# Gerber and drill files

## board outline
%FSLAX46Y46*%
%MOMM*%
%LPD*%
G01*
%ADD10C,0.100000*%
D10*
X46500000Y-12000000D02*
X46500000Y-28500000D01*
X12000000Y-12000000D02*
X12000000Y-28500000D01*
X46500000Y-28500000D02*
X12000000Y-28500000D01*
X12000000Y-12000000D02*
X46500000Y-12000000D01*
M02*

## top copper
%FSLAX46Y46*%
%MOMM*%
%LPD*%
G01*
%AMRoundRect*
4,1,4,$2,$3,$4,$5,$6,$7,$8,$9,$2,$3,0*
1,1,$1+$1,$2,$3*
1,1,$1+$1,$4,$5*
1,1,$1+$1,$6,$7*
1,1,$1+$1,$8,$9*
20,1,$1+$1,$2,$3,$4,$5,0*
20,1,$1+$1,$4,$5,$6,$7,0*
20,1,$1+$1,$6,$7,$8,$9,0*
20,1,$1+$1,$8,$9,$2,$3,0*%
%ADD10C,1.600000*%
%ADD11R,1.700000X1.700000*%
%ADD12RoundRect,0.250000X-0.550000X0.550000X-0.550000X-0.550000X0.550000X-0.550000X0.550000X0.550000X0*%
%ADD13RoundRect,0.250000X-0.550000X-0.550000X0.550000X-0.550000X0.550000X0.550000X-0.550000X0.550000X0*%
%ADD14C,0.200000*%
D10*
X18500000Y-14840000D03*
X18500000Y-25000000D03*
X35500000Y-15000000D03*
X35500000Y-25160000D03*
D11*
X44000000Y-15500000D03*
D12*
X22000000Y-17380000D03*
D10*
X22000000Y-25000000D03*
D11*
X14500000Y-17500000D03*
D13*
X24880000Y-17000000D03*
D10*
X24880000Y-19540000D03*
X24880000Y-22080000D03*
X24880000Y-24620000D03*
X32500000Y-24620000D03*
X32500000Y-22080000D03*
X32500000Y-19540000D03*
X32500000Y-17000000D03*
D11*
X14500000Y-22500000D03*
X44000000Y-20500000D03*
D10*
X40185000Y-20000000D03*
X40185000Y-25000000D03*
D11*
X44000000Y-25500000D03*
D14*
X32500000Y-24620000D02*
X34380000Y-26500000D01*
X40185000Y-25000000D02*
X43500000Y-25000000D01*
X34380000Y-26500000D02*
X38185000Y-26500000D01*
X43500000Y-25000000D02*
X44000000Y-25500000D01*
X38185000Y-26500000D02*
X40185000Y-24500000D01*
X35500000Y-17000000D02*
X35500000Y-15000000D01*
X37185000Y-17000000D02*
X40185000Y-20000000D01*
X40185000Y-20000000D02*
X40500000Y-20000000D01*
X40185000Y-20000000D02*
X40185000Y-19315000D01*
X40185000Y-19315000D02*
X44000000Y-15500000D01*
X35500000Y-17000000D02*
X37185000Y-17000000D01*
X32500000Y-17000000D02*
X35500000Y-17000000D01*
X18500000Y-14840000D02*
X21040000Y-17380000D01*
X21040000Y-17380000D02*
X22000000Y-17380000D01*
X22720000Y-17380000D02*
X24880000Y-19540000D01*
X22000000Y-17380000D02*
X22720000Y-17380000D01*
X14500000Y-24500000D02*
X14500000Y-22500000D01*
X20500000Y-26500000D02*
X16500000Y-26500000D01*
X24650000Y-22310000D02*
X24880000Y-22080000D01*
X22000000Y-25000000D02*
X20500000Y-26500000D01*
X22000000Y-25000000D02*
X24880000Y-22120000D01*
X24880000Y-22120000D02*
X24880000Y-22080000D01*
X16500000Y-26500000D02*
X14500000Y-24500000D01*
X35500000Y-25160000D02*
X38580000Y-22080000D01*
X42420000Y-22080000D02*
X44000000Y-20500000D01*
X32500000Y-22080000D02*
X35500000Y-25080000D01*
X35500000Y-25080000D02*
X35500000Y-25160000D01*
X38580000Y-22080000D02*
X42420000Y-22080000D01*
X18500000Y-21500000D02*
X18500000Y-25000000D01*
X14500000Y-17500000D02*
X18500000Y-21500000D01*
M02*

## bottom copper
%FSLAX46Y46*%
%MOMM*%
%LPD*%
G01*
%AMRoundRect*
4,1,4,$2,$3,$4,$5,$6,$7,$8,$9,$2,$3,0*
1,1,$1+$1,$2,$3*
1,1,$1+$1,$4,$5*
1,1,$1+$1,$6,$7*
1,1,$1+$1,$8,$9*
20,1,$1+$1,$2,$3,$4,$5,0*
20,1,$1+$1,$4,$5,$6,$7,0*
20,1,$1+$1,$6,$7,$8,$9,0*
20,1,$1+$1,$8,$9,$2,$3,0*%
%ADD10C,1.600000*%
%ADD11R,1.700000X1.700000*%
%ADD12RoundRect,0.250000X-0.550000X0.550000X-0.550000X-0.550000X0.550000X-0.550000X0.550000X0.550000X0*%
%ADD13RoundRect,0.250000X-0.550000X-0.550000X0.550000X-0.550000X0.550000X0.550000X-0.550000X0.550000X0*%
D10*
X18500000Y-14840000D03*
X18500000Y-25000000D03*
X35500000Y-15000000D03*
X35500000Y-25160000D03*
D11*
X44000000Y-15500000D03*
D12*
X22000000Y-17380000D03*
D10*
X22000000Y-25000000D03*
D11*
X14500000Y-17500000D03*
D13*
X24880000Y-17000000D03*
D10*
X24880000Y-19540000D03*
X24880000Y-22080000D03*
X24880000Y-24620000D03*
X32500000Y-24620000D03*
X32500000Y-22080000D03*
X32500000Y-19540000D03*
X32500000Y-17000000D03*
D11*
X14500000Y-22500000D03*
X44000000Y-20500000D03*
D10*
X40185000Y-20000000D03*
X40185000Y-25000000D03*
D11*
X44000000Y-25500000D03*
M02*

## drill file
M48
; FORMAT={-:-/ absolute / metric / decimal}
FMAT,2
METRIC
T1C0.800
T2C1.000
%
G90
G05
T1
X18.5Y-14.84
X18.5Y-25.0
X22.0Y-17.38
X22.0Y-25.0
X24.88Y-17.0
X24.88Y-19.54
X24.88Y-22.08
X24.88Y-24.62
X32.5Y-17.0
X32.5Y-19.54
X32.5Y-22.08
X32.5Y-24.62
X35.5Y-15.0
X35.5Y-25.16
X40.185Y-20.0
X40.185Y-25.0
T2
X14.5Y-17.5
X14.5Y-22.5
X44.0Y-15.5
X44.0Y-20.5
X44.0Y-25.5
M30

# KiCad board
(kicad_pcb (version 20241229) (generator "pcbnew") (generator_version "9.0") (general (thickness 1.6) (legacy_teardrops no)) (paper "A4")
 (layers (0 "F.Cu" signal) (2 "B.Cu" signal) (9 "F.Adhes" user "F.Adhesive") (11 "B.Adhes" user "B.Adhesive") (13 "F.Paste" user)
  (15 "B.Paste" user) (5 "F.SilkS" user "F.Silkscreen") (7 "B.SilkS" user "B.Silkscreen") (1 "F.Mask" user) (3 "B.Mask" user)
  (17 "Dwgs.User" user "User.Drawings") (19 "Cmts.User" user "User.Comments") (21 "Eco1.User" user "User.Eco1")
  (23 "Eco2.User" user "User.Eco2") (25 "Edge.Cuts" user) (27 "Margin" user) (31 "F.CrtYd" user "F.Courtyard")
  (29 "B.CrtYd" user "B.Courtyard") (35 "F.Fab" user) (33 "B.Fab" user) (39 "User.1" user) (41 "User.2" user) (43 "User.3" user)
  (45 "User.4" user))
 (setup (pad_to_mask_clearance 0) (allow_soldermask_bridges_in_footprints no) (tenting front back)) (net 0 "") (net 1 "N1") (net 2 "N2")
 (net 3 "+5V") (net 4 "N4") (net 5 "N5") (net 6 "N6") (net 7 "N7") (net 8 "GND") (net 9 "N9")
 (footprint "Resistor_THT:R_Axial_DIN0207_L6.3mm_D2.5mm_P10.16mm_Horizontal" (layer "F.Cu") (at 18.5 14.84 -90)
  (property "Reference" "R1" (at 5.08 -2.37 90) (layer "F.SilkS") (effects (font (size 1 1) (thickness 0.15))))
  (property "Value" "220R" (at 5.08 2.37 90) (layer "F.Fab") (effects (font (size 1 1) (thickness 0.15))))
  (pad "1" thru_hole circle (at 0 0 270) (size 1.6 1.6) (drill 0.8) (layers "*.Cu" "*.Mask") (remove_unused_layers no) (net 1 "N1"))
  (pad "2" thru_hole circle (at 10.16 0 270) (size 1.6 1.6) (drill 0.8) (layers "*.Cu" "*.Mask") (remove_unused_layers no) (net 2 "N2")))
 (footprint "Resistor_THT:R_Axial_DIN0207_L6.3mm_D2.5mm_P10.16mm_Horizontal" (layer "F.Cu") (at 35.5 15 -90)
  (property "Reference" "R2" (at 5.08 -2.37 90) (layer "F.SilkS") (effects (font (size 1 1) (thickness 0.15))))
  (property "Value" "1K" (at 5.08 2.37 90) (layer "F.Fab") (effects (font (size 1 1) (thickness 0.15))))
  (pad "1" thru_hole circle (at 0 0 270) (size 1.6 1.6) (drill 0.8) (layers "*.Cu" "*.Mask") (remove_unused_layers no) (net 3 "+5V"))
  (pad "2" thru_hole circle (at 10.16 0 270) (size 1.6 1.6) (drill 0.8) (layers "*.Cu" "*.Mask") (remove_unused_layers no) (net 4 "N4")))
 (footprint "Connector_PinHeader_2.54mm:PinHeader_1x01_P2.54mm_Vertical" (layer "F.Cu") (at 44 15.5)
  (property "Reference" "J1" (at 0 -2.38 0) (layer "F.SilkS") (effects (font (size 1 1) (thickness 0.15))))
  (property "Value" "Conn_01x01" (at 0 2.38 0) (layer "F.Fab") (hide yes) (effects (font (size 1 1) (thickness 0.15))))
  (pad "1" thru_hole rect (at 0 0) (size 1.7 1.7) (drill 1) (layers "*.Cu" "*.Mask") (remove_unused_layers no) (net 3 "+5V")))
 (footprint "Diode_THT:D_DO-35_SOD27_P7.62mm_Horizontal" (layer "F.Cu") (at 22 17.38 -90)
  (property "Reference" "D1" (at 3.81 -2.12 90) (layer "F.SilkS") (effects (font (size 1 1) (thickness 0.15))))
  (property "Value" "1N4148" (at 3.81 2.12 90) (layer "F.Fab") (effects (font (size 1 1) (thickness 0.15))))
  (pad "1" thru_hole roundrect (at 0 0 270) (size 1.6 1.6) (drill 0.8) (layers "*.Cu" "*.Mask") (remove_unused_layers no)
   (roundrect_rratio 0.15625) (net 1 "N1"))
  (pad "2" thru_hole circle (at 7.62 0 270) (size 1.6 1.6) (drill 0.8) (layers "*.Cu" "*.Mask") (remove_unused_layers no) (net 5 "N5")))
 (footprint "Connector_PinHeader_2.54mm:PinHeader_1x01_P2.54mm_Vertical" (layer "F.Cu") (at 14.5 17.5)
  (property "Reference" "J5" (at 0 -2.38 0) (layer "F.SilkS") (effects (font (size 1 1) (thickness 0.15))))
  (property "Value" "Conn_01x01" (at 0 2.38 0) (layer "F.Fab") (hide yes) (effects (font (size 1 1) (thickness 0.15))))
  (pad "1" thru_hole rect (at 0 0) (size 1.7 1.7) (drill 1) (layers "*.Cu" "*.Mask") (remove_unused_layers no) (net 2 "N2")))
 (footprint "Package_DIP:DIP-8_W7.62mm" (layer "F.Cu") (at 24.88 17)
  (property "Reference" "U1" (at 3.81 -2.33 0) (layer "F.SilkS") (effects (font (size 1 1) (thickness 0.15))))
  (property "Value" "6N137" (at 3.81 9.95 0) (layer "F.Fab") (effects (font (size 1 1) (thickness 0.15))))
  (pad "1" thru_hole roundrect (at 0 0) (size 1.6 1.6) (drill 0.8) (layers "*.Cu" "*.Mask") (remove_unused_layers no)
   (roundrect_rratio 0.15625) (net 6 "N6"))
  (pad "2" thru_hole circle (at 0 2.54) (size 1.6 1.6) (drill 0.8) (layers "*.Cu" "*.Mask") (remove_unused_layers no) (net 1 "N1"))
  (pad "3" thru_hole circle (at 0 5.08) (size 1.6 1.6) (drill 0.8) (layers "*.Cu" "*.Mask") (remove_unused_layers no) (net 5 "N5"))
  (pad "4" thru_hole circle (at 0 7.62) (size 1.6 1.6) (drill 0.8) (layers "*.Cu" "*.Mask") (remove_unused_layers no) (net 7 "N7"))
  (pad "5" thru_hole circle (at 7.62 7.62) (size 1.6 1.6) (drill 0.8) (layers "*.Cu" "*.Mask") (remove_unused_layers no) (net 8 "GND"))
  (pad "6" thru_hole circle (at 7.62 5.08) (size 1.6 1.6) (drill 0.8) (layers "*.Cu" "*.Mask") (remove_unused_layers no) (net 4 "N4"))
  (pad "7" thru_hole circle (at 7.62 2.54) (size 1.6 1.6) (drill 0.8) (layers "*.Cu" "*.Mask") (remove_unused_layers no) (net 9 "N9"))
  (pad "8" thru_hole circle (at 7.62 0) (size 1.6 1.6) (drill 0.8) (layers "*.Cu" "*.Mask") (remove_unused_layers no) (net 3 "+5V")))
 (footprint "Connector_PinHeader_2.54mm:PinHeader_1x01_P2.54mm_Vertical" (layer "F.Cu") (at 14.5 22.5)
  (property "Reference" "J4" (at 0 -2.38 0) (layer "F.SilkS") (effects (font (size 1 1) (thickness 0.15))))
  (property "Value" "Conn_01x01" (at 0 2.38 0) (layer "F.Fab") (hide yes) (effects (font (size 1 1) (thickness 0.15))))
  (pad "1" thru_hole rect (at 0 0) (size 1.7 1.7) (drill 1) (layers "*.Cu" "*.Mask") (remove_unused_layers no) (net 5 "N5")))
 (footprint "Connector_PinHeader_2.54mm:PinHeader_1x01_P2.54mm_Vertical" (layer "F.Cu") (at 44 20.5)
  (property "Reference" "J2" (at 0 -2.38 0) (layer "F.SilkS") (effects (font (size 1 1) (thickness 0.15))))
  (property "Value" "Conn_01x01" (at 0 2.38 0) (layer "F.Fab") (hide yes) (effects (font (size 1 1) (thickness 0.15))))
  (pad "1" thru_hole rect (at 0 0) (size 1.7 1.7) (drill 1) (layers "*.Cu" "*.Mask") (remove_unused_layers no) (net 4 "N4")))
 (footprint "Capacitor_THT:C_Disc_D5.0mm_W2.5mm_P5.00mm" (layer "F.Cu") (at 40.185 20 -90)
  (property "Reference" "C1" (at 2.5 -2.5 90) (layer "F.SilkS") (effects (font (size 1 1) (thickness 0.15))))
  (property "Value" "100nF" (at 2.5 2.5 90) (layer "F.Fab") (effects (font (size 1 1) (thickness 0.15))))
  (pad "1" thru_hole circle (at 0 0 270) (size 1.6 1.6) (drill 0.8) (layers "*.Cu" "*.Mask") (remove_unused_layers no) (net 3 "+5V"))
  (pad "2" thru_hole circle (at 5 0 270) (size 1.6 1.6) (drill 0.8) (layers "*.Cu" "*.Mask") (remove_unused_layers no) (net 8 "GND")))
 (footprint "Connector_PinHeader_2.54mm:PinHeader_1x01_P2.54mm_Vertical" (layer "F.Cu") (at 44 25.5)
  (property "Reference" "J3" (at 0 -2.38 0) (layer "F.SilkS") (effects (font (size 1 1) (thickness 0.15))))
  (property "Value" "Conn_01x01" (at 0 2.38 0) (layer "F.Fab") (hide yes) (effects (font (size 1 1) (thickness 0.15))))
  (pad "1" thru_hole rect (at 0 0) (size 1.7 1.7) (drill 1) (layers "*.Cu" "*.Mask") (remove_unused_layers no) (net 8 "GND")))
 (gr_line (start 46.5 12) (end 46.5 28.5) (stroke (width 0.1) (type default)) (layer "Edge.Cuts"))
 (gr_line (start 12 12) (end 12 28.5) (stroke (width 0.1) (type default)) (layer "Edge.Cuts"))
 (gr_line (start 46.5 28.5) (end 12 28.5) (stroke (width 0.1) (type default)) (layer "Edge.Cuts"))
 (gr_line (start 12 12) (end 46.5 12) (stroke (width 0.1) (type default)) (layer "Edge.Cuts"))
 (segment (start 32.5 24.62) (end 34.38 26.5) (width 0.2) (layer "F.Cu") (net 8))
 (segment (start 40.185 25) (end 43.5 25) (width 0.2) (layer "F.Cu") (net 8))
 (segment (start 34.38 26.5) (end 38.185 26.5) (width 0.2) (layer "F.Cu") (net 8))
 (segment (start 43.5 25) (end 44 25.5) (width 0.2) (layer "F.Cu") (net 8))
 (segment (start 38.185 26.5) (end 40.185 24.5) (width 0.2) (layer "F.Cu") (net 8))
 (segment (start 35.5 17) (end 35.5 15) (width 0.2) (layer "F.Cu") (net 3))
 (segment (start 37.185 17) (end 40.185 20) (width 0.2) (layer "F.Cu") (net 3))
 (segment (start 40.185 20) (end 40.5 20) (width 0.2) (layer "F.Cu") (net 3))
 (segment (start 40.185 20) (end 40.185 19.315) (width 0.2) (layer "F.Cu") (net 3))
 (segment (start 40.185 19.315) (end 44 15.5) (width 0.2) (layer "F.Cu") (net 3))
 (segment (start 35.5 17) (end 37.185 17) (width 0.2) (layer "F.Cu") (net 3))
 (segment (start 32.5 17) (end 35.5 17) (width 0.2) (layer "F.Cu") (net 3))
 (segment (start 18.5 14.84) (end 21.04 17.38) (width 0.2) (layer "F.Cu") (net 1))
 (segment (start 21.04 17.38) (end 22 17.38) (width 0.2) (layer "F.Cu") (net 1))
 (segment (start 22.72 17.38) (end 24.88 19.54) (width 0.2) (layer "F.Cu") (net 1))
 (segment (start 22 17.38) (end 22.72 17.38) (width 0.2) (layer "F.Cu") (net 1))
 (segment (start 14.5 24.5) (end 14.5 22.5) (width 0.2) (layer "F.Cu") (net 5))
 (segment (start 20.5 26.5) (end 16.5 26.5) (width 0.2) (layer "F.Cu") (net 5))
 (segment (start 24.65 22.31) (end 24.88 22.08) (width 0.2) (layer "F.Cu") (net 5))
 (segment (start 22 25) (end 20.5 26.5) (width 0.2) (layer "F.Cu") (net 5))
 (segment (start 22 25) (end 24.88 22.12) (width 0.2) (layer "F.Cu") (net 5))
 (segment (start 24.88 22.12) (end 24.88 22.08) (width 0.2) (layer "F.Cu") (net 5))
 (segment (start 16.5 26.5) (end 14.5 24.5) (width 0.2) (layer "F.Cu") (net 5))
 (segment (start 35.5 25.16) (end 38.58 22.08) (width 0.2) (layer "F.Cu") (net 4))
 (segment (start 42.42 22.08) (end 44 20.5) (width 0.2) (layer "F.Cu") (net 4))
 (segment (start 32.5 22.08) (end 35.5 25.08) (width 0.2) (layer "F.Cu") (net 4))
 (segment (start 35.5 25.08) (end 35.5 25.16) (width 0.2) (layer "F.Cu") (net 4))
 (segment (start 38.58 22.08) (end 42.42 22.08) (width 0.2) (layer "F.Cu") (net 4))
 (segment (start 18.5 21.5) (end 18.5 25) (width 0.2) (layer "F.Cu") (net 2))
 (segment (start 14.5 17.5) (end 18.5 21.5) (width 0.2) (layer "F.Cu") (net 2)))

